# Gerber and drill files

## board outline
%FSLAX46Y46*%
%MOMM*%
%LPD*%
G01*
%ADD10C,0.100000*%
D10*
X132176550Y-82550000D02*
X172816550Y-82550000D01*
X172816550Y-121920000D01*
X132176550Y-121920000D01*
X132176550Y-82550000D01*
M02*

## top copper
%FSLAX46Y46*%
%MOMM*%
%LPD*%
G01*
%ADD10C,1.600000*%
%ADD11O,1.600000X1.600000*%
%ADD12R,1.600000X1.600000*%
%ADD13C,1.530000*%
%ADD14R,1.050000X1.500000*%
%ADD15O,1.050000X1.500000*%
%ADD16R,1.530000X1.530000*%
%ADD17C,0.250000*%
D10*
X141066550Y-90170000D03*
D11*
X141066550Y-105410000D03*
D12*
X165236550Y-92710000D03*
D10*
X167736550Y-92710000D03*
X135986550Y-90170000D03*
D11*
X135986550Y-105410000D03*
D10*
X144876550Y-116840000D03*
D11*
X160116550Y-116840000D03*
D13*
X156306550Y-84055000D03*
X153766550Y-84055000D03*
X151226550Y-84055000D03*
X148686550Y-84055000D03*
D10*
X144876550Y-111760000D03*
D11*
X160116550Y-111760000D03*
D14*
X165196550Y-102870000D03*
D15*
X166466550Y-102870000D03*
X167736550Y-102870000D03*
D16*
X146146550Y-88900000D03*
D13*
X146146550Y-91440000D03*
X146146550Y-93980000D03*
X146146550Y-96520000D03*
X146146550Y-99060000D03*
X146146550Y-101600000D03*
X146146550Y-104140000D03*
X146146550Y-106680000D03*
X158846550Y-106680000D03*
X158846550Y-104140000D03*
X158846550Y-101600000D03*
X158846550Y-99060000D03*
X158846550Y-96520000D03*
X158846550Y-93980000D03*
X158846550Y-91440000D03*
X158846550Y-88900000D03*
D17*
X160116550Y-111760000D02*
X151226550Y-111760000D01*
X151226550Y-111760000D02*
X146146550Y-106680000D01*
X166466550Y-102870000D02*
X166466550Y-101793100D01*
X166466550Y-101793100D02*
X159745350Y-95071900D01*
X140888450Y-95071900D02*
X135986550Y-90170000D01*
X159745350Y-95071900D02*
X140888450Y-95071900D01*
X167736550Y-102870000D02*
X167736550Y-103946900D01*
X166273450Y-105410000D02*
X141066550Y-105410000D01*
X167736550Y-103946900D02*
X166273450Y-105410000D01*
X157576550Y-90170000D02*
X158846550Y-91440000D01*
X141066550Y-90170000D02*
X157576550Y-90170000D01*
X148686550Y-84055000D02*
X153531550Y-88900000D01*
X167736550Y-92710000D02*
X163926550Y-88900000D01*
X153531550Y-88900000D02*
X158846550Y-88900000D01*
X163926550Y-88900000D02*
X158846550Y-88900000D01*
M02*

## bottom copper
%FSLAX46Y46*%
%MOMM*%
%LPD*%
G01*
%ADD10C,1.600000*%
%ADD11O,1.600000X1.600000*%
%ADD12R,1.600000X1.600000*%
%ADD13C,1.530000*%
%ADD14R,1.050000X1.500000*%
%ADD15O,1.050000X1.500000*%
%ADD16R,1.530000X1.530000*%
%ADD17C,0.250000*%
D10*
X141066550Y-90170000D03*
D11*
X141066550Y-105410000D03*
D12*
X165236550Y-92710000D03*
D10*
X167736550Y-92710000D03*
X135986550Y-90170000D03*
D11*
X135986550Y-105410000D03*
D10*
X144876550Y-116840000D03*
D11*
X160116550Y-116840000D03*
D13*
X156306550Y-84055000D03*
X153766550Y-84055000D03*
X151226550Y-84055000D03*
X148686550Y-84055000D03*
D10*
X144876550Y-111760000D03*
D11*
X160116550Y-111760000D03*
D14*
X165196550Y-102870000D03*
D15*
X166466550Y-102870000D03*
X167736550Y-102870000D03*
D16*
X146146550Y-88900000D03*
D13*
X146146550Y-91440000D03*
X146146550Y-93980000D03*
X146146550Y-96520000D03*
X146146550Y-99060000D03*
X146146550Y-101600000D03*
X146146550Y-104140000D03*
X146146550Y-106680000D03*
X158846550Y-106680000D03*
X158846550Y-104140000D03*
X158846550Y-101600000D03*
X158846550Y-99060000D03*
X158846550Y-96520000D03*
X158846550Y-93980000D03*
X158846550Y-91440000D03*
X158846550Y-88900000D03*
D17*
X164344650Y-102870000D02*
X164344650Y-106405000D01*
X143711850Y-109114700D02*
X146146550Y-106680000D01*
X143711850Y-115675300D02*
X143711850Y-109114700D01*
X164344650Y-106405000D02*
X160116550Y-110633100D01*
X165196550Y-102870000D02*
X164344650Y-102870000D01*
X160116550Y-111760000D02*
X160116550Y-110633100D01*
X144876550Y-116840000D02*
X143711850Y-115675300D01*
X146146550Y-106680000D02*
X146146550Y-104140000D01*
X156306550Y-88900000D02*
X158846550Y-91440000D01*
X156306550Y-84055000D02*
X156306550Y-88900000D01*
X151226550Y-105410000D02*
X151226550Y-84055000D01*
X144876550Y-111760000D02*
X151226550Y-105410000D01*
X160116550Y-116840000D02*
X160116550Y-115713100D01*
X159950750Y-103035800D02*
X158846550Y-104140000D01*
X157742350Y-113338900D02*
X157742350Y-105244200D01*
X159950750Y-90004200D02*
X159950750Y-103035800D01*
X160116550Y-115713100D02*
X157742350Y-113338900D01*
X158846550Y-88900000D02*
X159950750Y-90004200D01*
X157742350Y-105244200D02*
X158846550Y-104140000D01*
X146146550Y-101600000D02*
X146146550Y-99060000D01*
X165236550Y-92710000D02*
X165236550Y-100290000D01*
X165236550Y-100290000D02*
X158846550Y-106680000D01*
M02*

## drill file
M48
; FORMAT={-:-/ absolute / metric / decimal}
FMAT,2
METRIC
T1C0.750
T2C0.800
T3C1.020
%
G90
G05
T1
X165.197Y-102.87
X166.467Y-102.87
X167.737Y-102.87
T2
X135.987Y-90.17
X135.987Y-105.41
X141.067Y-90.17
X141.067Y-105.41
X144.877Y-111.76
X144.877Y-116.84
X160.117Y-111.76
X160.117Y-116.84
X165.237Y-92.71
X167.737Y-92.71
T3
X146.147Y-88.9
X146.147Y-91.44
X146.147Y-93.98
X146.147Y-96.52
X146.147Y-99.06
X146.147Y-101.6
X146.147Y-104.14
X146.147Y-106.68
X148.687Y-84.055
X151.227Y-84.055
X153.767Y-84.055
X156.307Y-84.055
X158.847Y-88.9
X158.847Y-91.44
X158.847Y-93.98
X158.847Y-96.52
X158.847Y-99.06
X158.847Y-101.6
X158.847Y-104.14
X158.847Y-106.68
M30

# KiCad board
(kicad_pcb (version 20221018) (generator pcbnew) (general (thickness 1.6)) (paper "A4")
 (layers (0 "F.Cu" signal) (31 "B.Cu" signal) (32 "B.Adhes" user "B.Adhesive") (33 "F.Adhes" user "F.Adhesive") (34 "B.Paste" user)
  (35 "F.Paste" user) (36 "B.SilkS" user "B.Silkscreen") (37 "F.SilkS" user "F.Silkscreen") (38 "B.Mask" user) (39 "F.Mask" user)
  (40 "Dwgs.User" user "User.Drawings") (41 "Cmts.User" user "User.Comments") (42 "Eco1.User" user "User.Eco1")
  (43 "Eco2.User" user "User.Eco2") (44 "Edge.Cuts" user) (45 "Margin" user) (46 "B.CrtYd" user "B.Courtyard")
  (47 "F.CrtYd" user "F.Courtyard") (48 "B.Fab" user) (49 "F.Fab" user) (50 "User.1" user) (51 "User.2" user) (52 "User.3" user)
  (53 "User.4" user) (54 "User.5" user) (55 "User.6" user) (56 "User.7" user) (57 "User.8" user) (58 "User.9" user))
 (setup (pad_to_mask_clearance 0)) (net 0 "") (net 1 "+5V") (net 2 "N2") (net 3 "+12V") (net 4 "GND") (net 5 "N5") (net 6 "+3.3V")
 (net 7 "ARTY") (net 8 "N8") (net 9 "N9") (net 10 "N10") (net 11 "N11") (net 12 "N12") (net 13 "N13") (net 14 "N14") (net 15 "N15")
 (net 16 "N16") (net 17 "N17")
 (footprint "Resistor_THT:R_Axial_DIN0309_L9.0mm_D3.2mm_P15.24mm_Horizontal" (layer "F.Cu") (at 141.06655 90.17 -90)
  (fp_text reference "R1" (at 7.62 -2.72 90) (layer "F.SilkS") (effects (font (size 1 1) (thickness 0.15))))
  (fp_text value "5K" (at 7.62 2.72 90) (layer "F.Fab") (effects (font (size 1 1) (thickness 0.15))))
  (pad "1" thru_hole circle (at 0 0 270) (size 1.6 1.6) (drill 0.8) (layers "*.Cu" "*.Mask") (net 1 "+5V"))
  (pad "2" thru_hole oval (at 15.24 0 270) (size 1.6 1.6) (drill 0.8) (layers "*.Cu" "*.Mask") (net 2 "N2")))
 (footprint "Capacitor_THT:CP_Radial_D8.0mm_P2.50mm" (layer "F.Cu") (at 165.23655 92.71)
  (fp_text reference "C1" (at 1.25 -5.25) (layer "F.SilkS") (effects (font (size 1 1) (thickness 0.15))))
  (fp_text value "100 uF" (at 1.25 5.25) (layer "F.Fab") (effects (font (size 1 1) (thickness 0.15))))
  (pad "1" thru_hole rect (at 0 0) (size 1.6 1.6) (drill 0.8) (layers "*.Cu" "*.Mask") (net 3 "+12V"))
  (pad "2" thru_hole circle (at 2.5 0) (size 1.6 1.6) (drill 0.8) (layers "*.Cu" "*.Mask") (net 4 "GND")))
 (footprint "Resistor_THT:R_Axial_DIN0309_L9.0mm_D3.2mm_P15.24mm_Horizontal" (layer "F.Cu") (at 135.98655 90.17 -90)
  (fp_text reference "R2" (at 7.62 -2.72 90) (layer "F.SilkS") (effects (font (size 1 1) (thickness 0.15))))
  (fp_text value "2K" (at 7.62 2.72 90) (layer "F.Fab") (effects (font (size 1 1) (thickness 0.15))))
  (pad "1" thru_hole circle (at 0 0 270) (size 1.6 1.6) (drill 0.8) (layers "*.Cu" "*.Mask") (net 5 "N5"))
  (pad "2" thru_hole oval (at 15.24 0 270) (size 1.6 1.6) (drill 0.8) (layers "*.Cu" "*.Mask") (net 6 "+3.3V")))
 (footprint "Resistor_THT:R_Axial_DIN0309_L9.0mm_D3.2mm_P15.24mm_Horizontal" (layer "F.Cu") (at 144.87655 116.84)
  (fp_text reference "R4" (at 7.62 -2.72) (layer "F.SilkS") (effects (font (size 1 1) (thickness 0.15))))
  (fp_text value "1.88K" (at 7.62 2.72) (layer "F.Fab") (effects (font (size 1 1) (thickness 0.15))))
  (pad "1" thru_hole circle (at 0 0) (size 1.6 1.6) (drill 0.8) (layers "*.Cu" "*.Mask") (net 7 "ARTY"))
  (pad "2" thru_hole oval (at 15.24 0) (size 1.6 1.6) (drill 0.8) (layers "*.Cu" "*.Mask") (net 4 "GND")))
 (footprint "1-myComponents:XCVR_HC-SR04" (layer "F.Cu") (at 152.49655 84.055 180)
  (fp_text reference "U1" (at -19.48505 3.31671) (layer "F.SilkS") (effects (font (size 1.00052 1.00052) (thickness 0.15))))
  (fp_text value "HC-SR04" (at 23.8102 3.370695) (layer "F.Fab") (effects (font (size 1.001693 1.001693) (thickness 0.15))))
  (pad "1" thru_hole circle (at -3.81 0 180) (size 1.53 1.53) (drill 1.02) (layers "*.Cu" "*.Mask") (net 1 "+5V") (solder_mask_margin 0.102))
  (pad "2" thru_hole circle (at -1.27 0 180) (size 1.53 1.53) (drill 1.02) (layers "*.Cu" "*.Mask") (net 2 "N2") (solder_mask_margin 0.102))
  (pad "3" thru_hole circle (at 1.27 0 180) (size 1.53 1.53) (drill 1.02) (layers "*.Cu" "*.Mask") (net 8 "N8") (solder_mask_margin 0.102))
  (pad "4" thru_hole circle (at 3.81 0 180) (size 1.53 1.53) (drill 1.02) (layers "*.Cu" "*.Mask") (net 4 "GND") (solder_mask_margin 0.102)))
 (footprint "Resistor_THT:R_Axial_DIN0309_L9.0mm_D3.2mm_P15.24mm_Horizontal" (layer "F.Cu") (at 144.87655 111.76)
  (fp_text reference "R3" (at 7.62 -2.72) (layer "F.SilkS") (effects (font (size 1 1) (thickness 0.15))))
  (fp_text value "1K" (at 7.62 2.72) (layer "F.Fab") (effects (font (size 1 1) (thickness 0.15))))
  (pad "1" thru_hole circle (at 0 0) (size 1.6 1.6) (drill 0.8) (layers "*.Cu" "*.Mask") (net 8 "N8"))
  (pad "2" thru_hole oval (at 15.24 0) (size 1.6 1.6) (drill 0.8) (layers "*.Cu" "*.Mask") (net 7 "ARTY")))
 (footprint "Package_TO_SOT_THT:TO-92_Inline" (layer "F.Cu") (at 165.19655 102.87)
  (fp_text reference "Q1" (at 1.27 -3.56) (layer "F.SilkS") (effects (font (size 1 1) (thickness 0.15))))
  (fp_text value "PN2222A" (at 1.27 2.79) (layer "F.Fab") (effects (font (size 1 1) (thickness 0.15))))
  (pad "1" thru_hole rect (at 0 0) (size 1.05 1.5) (drill 0.75) (layers "*.Cu" "*.Mask") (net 7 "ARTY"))
  (pad "2" thru_hole oval (at 1.27 0) (size 1.05 1.5) (drill 0.75) (layers "*.Cu" "*.Mask") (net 5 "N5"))
  (pad "3" thru_hole oval (at 2.54 0) (size 1.05 1.5) (drill 0.75) (layers "*.Cu" "*.Mask") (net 2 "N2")))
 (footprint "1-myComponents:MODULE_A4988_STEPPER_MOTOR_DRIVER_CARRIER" (layer "F.Cu") (at 152.49655 97.79)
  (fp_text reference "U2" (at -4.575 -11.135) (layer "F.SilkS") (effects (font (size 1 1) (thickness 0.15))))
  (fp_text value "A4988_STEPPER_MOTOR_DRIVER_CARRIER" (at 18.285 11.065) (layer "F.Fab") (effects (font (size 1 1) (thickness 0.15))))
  (pad "1" thru_hole rect (at -6.35 -8.89) (size 1.53 1.53) (drill 1.02) (layers "*.Cu" "*.Mask") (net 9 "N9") (solder_mask_margin 0.102))
  (pad "2" thru_hole circle (at -6.35 -6.35) (size 1.53 1.53) (drill 1.02) (layers "*.Cu" "*.Mask") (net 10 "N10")
   (solder_mask_margin 0.102))
  (pad "3" thru_hole circle (at -6.35 -3.81) (size 1.53 1.53) (drill 1.02) (layers "*.Cu" "*.Mask") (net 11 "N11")
   (solder_mask_margin 0.102))
  (pad "4" thru_hole circle (at -6.35 -1.27) (size 1.53 1.53) (drill 1.02) (layers "*.Cu" "*.Mask") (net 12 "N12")
   (solder_mask_margin 0.102))
  (pad "5" thru_hole circle (at -6.35 1.27) (size 1.53 1.53) (drill 1.02) (layers "*.Cu" "*.Mask") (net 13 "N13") (solder_mask_margin 0.102))
  (pad "6" thru_hole circle (at -6.35 3.81) (size 1.53 1.53) (drill 1.02) (layers "*.Cu" "*.Mask") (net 13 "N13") (solder_mask_margin 0.102))
  (pad "7" thru_hole circle (at -6.35 6.35) (size 1.53 1.53) (drill 1.02) (layers "*.Cu" "*.Mask") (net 7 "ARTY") (solder_mask_margin 0.102))
  (pad "8" thru_hole circle (at -6.35 8.89) (size 1.53 1.53) (drill 1.02) (layers "*.Cu" "*.Mask") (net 7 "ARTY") (solder_mask_margin 0.102))
  (pad "9" thru_hole circle (at 6.35 8.89) (size 1.53 1.53) (drill 1.02) (layers "*.Cu" "*.Mask") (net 3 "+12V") (solder_mask_margin 0.102))
  (pad "10" thru_hole circle (at 6.35 6.35) (size 1.53 1.53) (drill 1.02) (layers "*.Cu" "*.Mask") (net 4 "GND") (solder_mask_margin 0.102))
  (pad "11" thru_hole circle (at 6.35 3.81) (size 1.53 1.53) (drill 1.02) (layers "*.Cu" "*.Mask") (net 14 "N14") (solder_mask_margin 0.102))
  (pad "12" thru_hole circle (at 6.35 1.27) (size 1.53 1.53) (drill 1.02) (layers "*.Cu" "*.Mask") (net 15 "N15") (solder_mask_margin 0.102))
  (pad "13" thru_hole circle (at 6.35 -1.27) (size 1.53 1.53) (drill 1.02) (layers "*.Cu" "*.Mask") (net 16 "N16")
   (solder_mask_margin 0.102))
  (pad "14" thru_hole circle (at 6.35 -3.81) (size 1.53 1.53) (drill 1.02) (layers "*.Cu" "*.Mask") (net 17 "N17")
   (solder_mask_margin 0.102))
  (pad "15" thru_hole circle (at 6.35 -6.35) (size 1.53 1.53) (drill 1.02) (layers "*.Cu" "*.Mask") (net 1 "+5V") (solder_mask_margin 0.102))
  (pad "16" thru_hole circle (at 6.35 -8.89) (size 1.53 1.53) (drill 1.02) (layers "*.Cu" "*.Mask") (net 4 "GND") (solder_mask_margin 0.102)))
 (gr_rect (start 132.17655 82.55) (end 172.81655 121.92) (stroke (width 0.1) (type default)) (fill none) (layer "Edge.Cuts"))
 (segment (start 160.11655 111.76) (end 151.22655 111.76) (width 0.25) (layer "F.Cu") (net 7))
 (segment (start 151.22655 111.76) (end 146.14655 106.68) (width 0.25) (layer "F.Cu") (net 7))
 (segment (start 164.34465 102.87) (end 164.34465 106.405) (width 0.25) (layer "B.Cu") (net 7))
 (segment (start 143.71185 109.1147) (end 146.14655 106.68) (width 0.25) (layer "B.Cu") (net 7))
 (segment (start 143.71185 115.6753) (end 143.71185 109.1147) (width 0.25) (layer "B.Cu") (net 7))
 (segment (start 164.34465 106.405) (end 160.11655 110.6331) (width 0.25) (layer "B.Cu") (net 7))
 (segment (start 165.19655 102.87) (end 164.34465 102.87) (width 0.25) (layer "B.Cu") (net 7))
 (segment (start 160.11655 111.76) (end 160.11655 110.6331) (width 0.25) (layer "B.Cu") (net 7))
 (segment (start 144.87655 116.84) (end 143.71185 115.6753) (width 0.25) (layer "B.Cu") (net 7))
 (segment (start 146.14655 106.68) (end 146.14655 104.14) (width 0.25) (layer "B.Cu") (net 7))
 (segment (start 166.46655 102.87) (end 166.46655 101.7931) (width 0.25) (layer "F.Cu") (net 5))
 (segment (start 166.46655 101.7931) (end 159.74535 95.0719) (width 0.25) (layer "F.Cu") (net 5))
 (segment (start 140.88845 95.0719) (end 135.98655 90.17) (width 0.25) (layer "F.Cu") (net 5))
 (segment (start 159.74535 95.0719) (end 140.88845 95.0719) (width 0.25) (layer "F.Cu") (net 5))
 (segment (start 167.73655 102.87) (end 167.73655 103.9469) (width 0.25) (layer "F.Cu") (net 2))
 (segment (start 166.27345 105.41) (end 141.06655 105.41) (width 0.25) (layer "F.Cu") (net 2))
 (segment (start 167.73655 103.9469) (end 166.27345 105.41) (width 0.25) (layer "F.Cu") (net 2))
 (segment (start 157.57655 90.17) (end 158.84655 91.44) (width 0.25) (layer "F.Cu") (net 1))
 (segment (start 141.06655 90.17) (end 157.57655 90.17) (width 0.25) (layer "F.Cu") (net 1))
 (segment (start 156.30655 88.9) (end 158.84655 91.44) (width 0.25) (layer "B.Cu") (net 1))
 (segment (start 156.30655 84.055) (end 156.30655 88.9) (width 0.25) (layer "B.Cu") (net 1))
 (segment (start 151.22655 105.41) (end 151.22655 84.055) (width 0.25) (layer "B.Cu") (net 8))
 (segment (start 144.87655 111.76) (end 151.22655 105.41) (width 0.25) (layer "B.Cu") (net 8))
 (segment (start 148.68655 84.055) (end 153.53155 88.9) (width 0.25) (layer "F.Cu") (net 4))
 (segment (start 167.73655 92.71) (end 163.92655 88.9) (width 0.25) (layer "F.Cu") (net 4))
 (segment (start 153.53155 88.9) (end 158.84655 88.9) (width 0.25) (layer "F.Cu") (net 4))
 (segment (start 163.92655 88.9) (end 158.84655 88.9) (width 0.25) (layer "F.Cu") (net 4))
 (segment (start 160.11655 116.84) (end 160.11655 115.7131) (width 0.25) (layer "B.Cu") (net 4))
 (segment (start 159.95075 103.0358) (end 158.84655 104.14) (width 0.25) (layer "B.Cu") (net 4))
 (segment (start 157.74235 113.3389) (end 157.74235 105.2442) (width 0.25) (layer "B.Cu") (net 4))
 (segment (start 159.95075 90.0042) (end 159.95075 103.0358) (width 0.25) (layer "B.Cu") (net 4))
 (segment (start 160.11655 115.7131) (end 157.74235 113.3389) (width 0.25) (layer "B.Cu") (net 4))
 (segment (start 158.84655 88.9) (end 159.95075 90.0042) (width 0.25) (layer "B.Cu") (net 4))
 (segment (start 157.74235 105.2442) (end 158.84655 104.14) (width 0.25) (layer "B.Cu") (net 4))
 (segment (start 146.14655 101.6) (end 146.14655 99.06) (width 0.25) (layer "B.Cu") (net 13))
 (segment (start 165.23655 92.71) (end 165.23655 100.29) (width 0.25) (layer "B.Cu") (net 3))
 (segment (start 165.23655 100.29) (end 158.84655 106.68) (width 0.25) (layer "B.Cu") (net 3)))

